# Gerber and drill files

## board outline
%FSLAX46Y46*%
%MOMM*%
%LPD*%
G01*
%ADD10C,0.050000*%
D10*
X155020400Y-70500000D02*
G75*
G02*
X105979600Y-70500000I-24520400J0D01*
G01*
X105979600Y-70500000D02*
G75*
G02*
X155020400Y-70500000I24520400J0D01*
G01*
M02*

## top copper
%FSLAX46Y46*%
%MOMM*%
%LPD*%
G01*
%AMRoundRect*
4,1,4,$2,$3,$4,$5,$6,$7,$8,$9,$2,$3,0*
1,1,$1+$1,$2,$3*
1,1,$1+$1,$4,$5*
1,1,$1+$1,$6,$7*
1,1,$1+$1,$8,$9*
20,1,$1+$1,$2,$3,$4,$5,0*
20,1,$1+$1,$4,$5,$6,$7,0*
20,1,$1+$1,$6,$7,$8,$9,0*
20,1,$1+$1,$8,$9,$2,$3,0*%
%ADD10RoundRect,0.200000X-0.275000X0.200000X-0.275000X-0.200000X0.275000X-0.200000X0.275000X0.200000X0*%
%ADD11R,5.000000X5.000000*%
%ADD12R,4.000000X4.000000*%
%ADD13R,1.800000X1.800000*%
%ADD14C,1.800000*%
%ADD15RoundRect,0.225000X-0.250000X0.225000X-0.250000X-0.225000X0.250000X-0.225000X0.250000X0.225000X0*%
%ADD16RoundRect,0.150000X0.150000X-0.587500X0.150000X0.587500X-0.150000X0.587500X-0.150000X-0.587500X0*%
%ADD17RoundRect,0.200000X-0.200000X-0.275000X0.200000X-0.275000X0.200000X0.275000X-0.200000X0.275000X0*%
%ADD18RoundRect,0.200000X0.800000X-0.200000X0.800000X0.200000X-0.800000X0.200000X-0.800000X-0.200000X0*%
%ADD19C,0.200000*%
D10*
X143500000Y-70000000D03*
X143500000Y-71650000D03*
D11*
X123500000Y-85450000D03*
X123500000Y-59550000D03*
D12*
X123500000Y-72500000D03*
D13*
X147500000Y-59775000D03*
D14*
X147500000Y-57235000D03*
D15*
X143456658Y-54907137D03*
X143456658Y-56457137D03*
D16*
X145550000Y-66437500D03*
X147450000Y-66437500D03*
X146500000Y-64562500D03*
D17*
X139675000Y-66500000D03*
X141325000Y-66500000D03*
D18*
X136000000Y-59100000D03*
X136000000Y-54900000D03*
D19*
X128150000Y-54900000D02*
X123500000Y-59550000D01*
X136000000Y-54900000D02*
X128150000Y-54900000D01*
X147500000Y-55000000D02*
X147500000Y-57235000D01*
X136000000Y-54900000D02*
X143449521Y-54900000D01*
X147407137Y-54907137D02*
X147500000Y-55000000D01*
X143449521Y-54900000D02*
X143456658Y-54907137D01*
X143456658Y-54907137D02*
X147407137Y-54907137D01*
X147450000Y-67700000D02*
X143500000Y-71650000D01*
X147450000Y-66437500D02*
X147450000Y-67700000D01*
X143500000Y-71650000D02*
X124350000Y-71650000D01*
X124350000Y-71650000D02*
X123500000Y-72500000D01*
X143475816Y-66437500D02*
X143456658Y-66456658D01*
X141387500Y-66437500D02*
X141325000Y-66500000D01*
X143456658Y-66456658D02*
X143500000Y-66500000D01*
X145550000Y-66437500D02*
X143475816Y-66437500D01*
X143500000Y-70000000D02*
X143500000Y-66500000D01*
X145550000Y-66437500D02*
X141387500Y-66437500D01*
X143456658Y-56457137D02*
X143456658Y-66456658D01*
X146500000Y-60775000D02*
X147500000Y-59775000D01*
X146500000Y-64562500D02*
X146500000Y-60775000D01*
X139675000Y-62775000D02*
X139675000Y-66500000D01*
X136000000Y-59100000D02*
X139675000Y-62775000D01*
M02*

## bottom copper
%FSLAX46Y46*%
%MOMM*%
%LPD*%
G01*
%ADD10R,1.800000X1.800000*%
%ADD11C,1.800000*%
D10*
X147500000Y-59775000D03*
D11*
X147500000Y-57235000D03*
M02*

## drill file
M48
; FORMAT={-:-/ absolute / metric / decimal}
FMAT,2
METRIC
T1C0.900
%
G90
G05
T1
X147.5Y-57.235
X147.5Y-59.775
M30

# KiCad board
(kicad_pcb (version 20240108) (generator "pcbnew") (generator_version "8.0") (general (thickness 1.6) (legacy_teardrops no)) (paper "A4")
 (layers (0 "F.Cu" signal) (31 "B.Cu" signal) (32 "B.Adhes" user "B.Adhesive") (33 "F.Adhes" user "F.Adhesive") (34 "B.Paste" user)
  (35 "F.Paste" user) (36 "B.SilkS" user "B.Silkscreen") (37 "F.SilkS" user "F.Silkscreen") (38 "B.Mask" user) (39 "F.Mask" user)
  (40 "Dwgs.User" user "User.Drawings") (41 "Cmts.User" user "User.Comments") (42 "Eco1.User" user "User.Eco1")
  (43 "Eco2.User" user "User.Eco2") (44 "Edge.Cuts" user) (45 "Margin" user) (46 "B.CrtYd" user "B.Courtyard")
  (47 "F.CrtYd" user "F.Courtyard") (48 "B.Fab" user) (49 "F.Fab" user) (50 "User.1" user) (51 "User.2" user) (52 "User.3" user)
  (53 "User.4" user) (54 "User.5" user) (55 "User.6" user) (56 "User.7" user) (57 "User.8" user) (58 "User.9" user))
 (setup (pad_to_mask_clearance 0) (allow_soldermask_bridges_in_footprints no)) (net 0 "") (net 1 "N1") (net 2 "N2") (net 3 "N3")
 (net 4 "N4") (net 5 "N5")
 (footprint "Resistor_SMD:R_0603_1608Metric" (layer "F.Cu") (at 143.5 70.825 -90)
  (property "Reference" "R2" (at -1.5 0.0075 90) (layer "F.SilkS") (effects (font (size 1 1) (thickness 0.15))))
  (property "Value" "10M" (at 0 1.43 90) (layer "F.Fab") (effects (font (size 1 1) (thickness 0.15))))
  (pad "1" smd roundrect (at -0.825 0 270) (size 0.8 0.95) (layers "F.Cu" "F.Paste" "F.Mask") (roundrect_rratio 0.25) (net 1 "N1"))
  (pad "2" smd roundrect (at 0.825 0 270) (size 0.8 0.95) (layers "F.Cu" "F.Paste" "F.Mask") (roundrect_rratio 0.25) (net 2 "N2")))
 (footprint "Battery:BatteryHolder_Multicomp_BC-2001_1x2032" (layer "F.Cu") (at 123.5 72.5 90)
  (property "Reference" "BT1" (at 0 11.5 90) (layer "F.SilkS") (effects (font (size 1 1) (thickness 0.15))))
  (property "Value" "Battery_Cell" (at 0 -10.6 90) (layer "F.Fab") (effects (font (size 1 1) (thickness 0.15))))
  (pad "1" smd rect (at -12.95 0 90) (size 5 5) (layers "F.Cu" "F.Paste" "F.Mask") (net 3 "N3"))
  (pad "1" smd rect (at 12.95 0 90) (size 5 5) (layers "F.Cu" "F.Paste" "F.Mask") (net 3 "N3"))
  (pad "2" smd rect (at 0 0 90) (size 4 4) (layers "F.Cu" "F.Paste" "F.Mask") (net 2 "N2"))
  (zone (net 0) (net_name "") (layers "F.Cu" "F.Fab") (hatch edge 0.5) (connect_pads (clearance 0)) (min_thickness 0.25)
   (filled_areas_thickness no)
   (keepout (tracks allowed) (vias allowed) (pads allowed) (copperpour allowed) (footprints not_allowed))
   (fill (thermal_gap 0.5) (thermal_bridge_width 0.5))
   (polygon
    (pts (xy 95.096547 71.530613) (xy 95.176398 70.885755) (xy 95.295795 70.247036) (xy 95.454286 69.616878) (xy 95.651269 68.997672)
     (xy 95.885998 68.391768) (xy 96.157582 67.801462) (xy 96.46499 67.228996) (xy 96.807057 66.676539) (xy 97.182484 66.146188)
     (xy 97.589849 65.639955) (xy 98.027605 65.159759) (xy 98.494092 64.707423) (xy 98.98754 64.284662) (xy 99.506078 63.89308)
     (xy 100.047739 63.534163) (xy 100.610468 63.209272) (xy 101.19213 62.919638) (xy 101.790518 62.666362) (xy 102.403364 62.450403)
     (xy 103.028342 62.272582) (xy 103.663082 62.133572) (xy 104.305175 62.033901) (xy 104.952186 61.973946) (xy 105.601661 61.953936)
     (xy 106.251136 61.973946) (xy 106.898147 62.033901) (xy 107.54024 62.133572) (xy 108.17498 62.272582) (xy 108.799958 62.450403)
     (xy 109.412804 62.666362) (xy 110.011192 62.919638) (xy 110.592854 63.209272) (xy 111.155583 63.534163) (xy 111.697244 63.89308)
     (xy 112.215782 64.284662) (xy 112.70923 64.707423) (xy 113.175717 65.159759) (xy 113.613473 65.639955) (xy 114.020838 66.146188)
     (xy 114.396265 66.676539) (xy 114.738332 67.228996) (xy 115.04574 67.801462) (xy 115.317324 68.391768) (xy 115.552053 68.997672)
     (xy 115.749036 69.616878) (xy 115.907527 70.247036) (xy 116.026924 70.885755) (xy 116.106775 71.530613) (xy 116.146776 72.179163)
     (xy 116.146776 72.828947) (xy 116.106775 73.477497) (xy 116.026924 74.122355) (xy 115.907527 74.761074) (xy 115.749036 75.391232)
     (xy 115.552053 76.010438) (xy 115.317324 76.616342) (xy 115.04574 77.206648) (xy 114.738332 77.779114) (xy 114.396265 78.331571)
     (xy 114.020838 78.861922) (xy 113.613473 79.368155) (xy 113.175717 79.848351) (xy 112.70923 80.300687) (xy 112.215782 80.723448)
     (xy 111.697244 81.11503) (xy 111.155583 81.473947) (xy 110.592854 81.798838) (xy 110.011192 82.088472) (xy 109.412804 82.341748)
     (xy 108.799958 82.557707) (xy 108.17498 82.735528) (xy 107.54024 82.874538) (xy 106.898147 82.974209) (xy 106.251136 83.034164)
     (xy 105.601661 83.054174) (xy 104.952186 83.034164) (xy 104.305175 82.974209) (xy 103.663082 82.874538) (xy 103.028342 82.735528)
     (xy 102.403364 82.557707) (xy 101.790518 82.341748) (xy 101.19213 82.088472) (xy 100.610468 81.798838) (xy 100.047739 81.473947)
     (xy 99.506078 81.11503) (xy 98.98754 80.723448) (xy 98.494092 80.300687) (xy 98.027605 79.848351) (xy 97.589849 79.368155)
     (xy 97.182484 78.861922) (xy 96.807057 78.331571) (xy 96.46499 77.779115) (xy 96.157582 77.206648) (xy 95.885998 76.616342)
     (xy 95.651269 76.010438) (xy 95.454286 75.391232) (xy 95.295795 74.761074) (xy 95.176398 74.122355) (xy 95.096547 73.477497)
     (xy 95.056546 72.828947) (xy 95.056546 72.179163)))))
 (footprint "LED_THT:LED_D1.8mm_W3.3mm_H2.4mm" (layer "F.Cu") (at 147.5 59.775 90)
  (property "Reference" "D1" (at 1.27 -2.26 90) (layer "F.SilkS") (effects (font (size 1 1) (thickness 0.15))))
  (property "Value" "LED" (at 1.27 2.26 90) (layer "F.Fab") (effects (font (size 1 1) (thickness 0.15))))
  (pad "1" thru_hole rect (at 0 0 90) (size 1.8 1.8) (drill 0.9) (layers "*.Cu" "*.Mask") (remove_unused_layers no) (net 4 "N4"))
  (pad "2" thru_hole circle (at 2.54 0 90) (size 1.8 1.8) (drill 0.9) (layers "*.Cu" "*.Mask") (remove_unused_layers no) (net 3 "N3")))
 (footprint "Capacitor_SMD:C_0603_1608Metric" (layer "F.Cu") (at 143.456658 55.682137 -90)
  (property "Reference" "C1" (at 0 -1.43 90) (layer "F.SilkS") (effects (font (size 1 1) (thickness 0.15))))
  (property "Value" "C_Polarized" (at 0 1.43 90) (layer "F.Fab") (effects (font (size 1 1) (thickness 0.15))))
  (pad "1" smd roundrect (at -0.775 0 270) (size 0.9 0.95) (layers "F.Cu" "F.Paste" "F.Mask") (roundrect_rratio 0.25) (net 3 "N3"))
  (pad "2" smd roundrect (at 0.775 0 270) (size 0.9 0.95) (layers "F.Cu" "F.Paste" "F.Mask") (roundrect_rratio 0.25) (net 1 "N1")))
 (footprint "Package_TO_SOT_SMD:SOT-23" (layer "F.Cu") (at 146.5 65.5 90)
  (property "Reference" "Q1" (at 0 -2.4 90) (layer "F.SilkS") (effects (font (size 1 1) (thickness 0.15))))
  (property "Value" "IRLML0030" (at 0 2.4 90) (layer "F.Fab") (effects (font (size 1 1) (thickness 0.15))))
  (pad "1" smd roundrect (at -0.9375 -0.95 90) (size 1.475 0.6) (layers "F.Cu" "F.Paste" "F.Mask") (roundrect_rratio 0.25) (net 1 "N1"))
  (pad "2" smd roundrect (at -0.9375 0.95 90) (size 1.475 0.6) (layers "F.Cu" "F.Paste" "F.Mask") (roundrect_rratio 0.25) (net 2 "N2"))
  (pad "3" smd roundrect (at 0.9375 0 90) (size 1.475 0.6) (layers "F.Cu" "F.Paste" "F.Mask") (roundrect_rratio 0.25) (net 4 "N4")))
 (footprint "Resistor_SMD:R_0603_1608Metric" (layer "F.Cu") (at 140.5 66.5)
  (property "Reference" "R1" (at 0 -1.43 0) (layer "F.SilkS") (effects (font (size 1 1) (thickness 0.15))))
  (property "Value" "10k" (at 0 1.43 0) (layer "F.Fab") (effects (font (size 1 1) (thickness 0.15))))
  (pad "1" smd roundrect (at -0.825 0) (size 0.8 0.95) (layers "F.Cu" "F.Paste" "F.Mask") (roundrect_rratio 0.25) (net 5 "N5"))
  (pad "2" smd roundrect (at 0.825 0) (size 0.8 0.95) (layers "F.Cu" "F.Paste" "F.Mask") (roundrect_rratio 0.25) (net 1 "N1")))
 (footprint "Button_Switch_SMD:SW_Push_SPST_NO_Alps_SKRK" (layer "F.Cu") (at 136 57 90)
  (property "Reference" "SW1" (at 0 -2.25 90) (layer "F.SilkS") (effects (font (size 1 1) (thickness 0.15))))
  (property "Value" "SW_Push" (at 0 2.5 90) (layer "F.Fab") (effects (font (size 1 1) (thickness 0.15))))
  (pad "1" smd roundrect (at -2.1 0 90) (size 0.8 2) (layers "F.Cu" "F.Paste" "F.Mask") (roundrect_rratio 0.25) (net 5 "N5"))
  (pad "2" smd roundrect (at 2.1 0 90) (size 0.8 2) (layers "F.Cu" "F.Paste" "F.Mask") (roundrect_rratio 0.25) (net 3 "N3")))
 (gr_circle (center 130.5 70.5) (end 153.5 79) (stroke (width 0.05) (type default)) (fill none) (layer "Edge.Cuts"))
 (segment (start 128.15 54.9) (end 123.5 59.55) (width 0.2) (layer "F.Cu") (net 3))
 (segment (start 136 54.9) (end 128.15 54.9) (width 0.2) (layer "F.Cu") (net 3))
 (segment (start 147.5 55) (end 147.5 57.235) (width 0.2) (layer "F.Cu") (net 3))
 (segment (start 136 54.9) (end 143.449521 54.9) (width 0.2) (layer "F.Cu") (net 3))
 (segment (start 147.407137 54.907137) (end 147.5 55) (width 0.2) (layer "F.Cu") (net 3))
 (segment (start 143.449521 54.9) (end 143.456658 54.907137) (width 0.2) (layer "F.Cu") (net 3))
 (segment (start 143.456658 54.907137) (end 147.407137 54.907137) (width 0.2) (layer "F.Cu") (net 3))
 (segment (start 147.45 67.7) (end 143.5 71.65) (width 0.2) (layer "F.Cu") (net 2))
 (segment (start 147.45 66.4375) (end 147.45 67.7) (width 0.2) (layer "F.Cu") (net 2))
 (segment (start 143.5 71.65) (end 124.35 71.65) (width 0.2) (layer "F.Cu") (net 2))
 (segment (start 124.35 71.65) (end 123.5 72.5) (width 0.2) (layer "F.Cu") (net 2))
 (segment (start 143.475816 66.4375) (end 143.456658 66.456658) (width 0.2) (layer "F.Cu") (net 1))
 (segment (start 141.3875 66.4375) (end 141.325 66.5) (width 0.2) (layer "F.Cu") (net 1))
 (segment (start 143.456658 66.456658) (end 143.5 66.5) (width 0.2) (layer "F.Cu") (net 1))
 (segment (start 145.55 66.4375) (end 143.475816 66.4375) (width 0.2) (layer "F.Cu") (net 1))
 (segment (start 143.5 70) (end 143.5 66.5) (width 0.2) (layer "F.Cu") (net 1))
 (segment (start 145.55 66.4375) (end 141.3875 66.4375) (width 0.2) (layer "F.Cu") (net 1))
 (segment (start 143.456658 56.457137) (end 143.456658 66.456658) (width 0.2) (layer "F.Cu") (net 1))
 (segment (start 146.5 60.775) (end 147.5 59.775) (width 0.2) (layer "F.Cu") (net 4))
 (segment (start 146.5 64.5625) (end 146.5 60.775) (width 0.2) (layer "F.Cu") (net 4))
 (segment (start 139.675 62.775) (end 139.675 66.5) (width 0.2) (layer "F.Cu") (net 5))
 (segment (start 136 59.1) (end 139.675 62.775) (width 0.2) (layer "F.Cu") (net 5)))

